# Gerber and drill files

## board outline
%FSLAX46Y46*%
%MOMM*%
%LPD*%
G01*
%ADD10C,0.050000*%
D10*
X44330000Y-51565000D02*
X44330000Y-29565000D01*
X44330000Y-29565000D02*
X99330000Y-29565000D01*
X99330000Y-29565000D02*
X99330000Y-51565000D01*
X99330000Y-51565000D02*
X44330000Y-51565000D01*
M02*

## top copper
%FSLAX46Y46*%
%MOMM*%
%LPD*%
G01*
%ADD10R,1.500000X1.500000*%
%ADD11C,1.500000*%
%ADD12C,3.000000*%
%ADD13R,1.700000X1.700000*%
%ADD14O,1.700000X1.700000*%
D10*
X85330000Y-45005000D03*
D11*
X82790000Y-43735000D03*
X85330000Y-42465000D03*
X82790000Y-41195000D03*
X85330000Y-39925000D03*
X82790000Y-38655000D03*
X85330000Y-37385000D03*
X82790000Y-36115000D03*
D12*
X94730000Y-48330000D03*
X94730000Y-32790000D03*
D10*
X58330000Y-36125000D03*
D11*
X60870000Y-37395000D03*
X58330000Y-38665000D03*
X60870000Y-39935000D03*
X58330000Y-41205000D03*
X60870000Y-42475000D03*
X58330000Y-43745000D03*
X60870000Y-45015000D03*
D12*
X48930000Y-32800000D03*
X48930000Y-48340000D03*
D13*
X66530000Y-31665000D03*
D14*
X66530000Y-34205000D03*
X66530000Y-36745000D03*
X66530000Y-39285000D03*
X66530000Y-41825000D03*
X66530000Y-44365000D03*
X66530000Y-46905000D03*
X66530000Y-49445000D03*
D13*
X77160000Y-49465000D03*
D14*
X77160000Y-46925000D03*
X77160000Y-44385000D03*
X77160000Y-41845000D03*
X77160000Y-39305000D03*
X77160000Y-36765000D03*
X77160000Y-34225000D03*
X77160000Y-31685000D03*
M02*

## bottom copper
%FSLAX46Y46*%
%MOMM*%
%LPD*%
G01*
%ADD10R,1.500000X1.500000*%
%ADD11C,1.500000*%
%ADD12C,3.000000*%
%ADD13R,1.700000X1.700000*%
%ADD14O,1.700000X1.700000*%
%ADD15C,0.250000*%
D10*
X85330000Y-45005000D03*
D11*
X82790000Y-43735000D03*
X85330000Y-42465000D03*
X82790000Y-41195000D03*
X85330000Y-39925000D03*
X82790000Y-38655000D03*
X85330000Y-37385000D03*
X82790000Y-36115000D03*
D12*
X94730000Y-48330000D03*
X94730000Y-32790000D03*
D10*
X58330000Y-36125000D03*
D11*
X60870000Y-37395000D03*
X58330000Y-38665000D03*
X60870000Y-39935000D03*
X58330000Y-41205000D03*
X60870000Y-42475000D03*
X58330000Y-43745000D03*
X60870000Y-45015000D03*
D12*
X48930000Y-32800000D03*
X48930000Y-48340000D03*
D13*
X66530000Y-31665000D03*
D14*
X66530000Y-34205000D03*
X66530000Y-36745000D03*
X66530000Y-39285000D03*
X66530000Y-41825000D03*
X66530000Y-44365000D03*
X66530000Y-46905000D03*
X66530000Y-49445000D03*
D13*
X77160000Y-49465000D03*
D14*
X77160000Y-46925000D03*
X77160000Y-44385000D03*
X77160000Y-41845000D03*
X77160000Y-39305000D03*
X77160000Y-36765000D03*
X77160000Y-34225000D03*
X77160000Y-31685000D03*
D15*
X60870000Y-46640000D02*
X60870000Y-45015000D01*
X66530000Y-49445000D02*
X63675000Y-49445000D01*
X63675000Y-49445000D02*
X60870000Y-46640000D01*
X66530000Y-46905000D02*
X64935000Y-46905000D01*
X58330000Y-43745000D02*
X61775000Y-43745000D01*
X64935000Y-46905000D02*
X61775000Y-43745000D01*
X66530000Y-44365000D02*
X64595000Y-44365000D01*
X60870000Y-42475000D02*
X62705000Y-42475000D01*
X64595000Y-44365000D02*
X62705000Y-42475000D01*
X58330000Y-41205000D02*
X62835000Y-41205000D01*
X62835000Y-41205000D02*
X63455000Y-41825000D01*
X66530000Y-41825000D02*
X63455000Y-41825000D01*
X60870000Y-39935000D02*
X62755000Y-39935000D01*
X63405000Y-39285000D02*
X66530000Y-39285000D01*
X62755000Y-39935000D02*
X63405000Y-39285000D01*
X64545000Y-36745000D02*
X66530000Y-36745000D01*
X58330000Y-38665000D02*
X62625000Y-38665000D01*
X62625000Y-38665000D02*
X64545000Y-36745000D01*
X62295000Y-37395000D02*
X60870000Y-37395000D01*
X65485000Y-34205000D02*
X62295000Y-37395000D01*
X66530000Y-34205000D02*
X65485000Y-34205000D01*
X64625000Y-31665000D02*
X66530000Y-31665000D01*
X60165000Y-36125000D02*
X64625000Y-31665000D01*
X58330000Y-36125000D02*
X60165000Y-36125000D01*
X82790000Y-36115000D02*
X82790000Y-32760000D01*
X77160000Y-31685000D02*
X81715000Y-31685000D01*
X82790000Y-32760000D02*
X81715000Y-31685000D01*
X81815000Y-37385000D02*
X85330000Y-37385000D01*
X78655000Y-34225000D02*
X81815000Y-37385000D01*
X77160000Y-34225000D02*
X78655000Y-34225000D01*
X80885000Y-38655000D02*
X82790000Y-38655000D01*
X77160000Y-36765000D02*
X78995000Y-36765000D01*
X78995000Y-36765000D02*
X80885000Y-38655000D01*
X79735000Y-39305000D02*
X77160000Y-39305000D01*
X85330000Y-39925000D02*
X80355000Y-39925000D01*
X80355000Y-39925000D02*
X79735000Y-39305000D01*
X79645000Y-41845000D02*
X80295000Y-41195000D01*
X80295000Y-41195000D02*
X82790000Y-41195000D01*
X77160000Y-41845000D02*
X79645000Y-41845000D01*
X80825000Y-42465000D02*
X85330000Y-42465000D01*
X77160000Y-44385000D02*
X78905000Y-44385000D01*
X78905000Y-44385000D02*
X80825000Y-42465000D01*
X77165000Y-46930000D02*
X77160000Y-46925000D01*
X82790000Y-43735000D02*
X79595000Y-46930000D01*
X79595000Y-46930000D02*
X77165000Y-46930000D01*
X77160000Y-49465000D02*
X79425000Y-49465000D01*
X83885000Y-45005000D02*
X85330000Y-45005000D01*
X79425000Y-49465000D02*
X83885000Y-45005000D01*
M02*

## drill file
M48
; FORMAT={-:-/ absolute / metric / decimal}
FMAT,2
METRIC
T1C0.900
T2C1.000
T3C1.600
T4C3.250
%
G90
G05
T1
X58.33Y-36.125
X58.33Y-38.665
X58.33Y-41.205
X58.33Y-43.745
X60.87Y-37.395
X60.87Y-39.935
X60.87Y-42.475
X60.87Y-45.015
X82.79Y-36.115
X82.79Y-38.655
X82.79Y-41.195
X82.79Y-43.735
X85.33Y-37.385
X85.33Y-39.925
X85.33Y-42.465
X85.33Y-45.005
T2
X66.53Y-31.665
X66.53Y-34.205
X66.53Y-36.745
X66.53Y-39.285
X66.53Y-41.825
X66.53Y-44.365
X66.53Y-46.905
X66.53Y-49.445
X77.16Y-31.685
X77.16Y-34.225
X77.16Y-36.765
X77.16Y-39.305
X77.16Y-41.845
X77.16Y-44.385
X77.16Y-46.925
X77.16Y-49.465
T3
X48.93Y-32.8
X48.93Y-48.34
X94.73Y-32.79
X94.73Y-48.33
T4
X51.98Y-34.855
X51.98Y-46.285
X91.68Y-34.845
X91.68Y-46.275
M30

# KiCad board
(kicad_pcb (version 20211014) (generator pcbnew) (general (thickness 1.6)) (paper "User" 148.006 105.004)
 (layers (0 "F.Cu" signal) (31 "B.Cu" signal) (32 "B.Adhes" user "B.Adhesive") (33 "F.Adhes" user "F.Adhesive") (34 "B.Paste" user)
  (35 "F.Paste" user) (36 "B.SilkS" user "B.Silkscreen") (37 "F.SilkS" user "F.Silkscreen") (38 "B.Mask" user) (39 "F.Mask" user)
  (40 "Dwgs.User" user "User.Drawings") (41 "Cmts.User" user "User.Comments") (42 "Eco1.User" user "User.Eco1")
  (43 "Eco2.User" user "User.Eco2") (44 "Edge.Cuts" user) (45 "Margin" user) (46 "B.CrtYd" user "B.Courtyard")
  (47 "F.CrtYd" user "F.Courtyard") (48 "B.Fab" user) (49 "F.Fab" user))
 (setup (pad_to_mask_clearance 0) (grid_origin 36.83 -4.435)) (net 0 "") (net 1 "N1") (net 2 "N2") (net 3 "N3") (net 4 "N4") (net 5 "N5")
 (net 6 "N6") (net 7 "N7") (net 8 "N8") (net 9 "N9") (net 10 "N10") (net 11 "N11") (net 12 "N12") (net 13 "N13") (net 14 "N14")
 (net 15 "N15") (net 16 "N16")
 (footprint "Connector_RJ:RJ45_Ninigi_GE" (layer "F.Cu") (at 85.33 45.005 90)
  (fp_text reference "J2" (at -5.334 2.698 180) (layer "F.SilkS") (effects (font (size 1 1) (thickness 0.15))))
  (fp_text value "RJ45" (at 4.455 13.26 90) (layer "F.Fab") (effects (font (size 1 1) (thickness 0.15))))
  (pad "" np_thru_hole circle locked (at -1.27 6.35 90) (size 3.25 3.25) (drill 3.25) (layers *.Cu *.Mask))
  (pad "" np_thru_hole circle locked (at 10.16 6.35 270) (size 3.25 3.25) (drill 3.25) (layers *.Cu *.Mask))
  (pad "1" thru_hole rect locked (at 0 0 270) (size 1.5 1.5) (drill 0.9) (layers *.Cu *.Mask) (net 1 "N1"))
  (pad "2" thru_hole circle locked (at 1.27 -2.54 270) (size 1.5 1.5) (drill 0.9) (layers *.Cu *.Mask) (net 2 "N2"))
  (pad "3" thru_hole circle locked (at 2.54 0 270) (size 1.5 1.5) (drill 0.9) (layers *.Cu *.Mask) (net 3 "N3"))
  (pad "4" thru_hole circle locked (at 3.81 -2.54 270) (size 1.5 1.5) (drill 0.9) (layers *.Cu *.Mask) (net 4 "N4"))
  (pad "5" thru_hole circle locked (at 5.08 0 270) (size 1.5 1.5) (drill 0.9) (layers *.Cu *.Mask) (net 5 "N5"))
  (pad "6" thru_hole circle locked (at 6.35 -2.54 270) (size 1.5 1.5) (drill 0.9) (layers *.Cu *.Mask) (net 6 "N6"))
  (pad "7" thru_hole circle locked (at 7.62 0 270) (size 1.5 1.5) (drill 0.9) (layers *.Cu *.Mask) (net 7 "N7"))
  (pad "8" thru_hole circle locked (at 8.89 -2.54 270) (size 1.5 1.5) (drill 0.9) (layers *.Cu *.Mask) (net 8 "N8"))
  (pad "SH" thru_hole circle locked (at -3.325 9.4 90) (size 3 3) (drill 1.6) (layers *.Cu *.Mask))
  (pad "SH" thru_hole circle locked (at 12.215 9.4 270) (size 3 3) (drill 1.6) (layers *.Cu *.Mask)))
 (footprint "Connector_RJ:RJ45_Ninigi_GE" (layer "F.Cu") (at 58.33 36.125 -90)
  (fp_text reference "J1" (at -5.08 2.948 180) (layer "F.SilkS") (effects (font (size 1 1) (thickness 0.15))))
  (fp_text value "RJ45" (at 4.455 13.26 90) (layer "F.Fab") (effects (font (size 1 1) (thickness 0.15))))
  (pad "" np_thru_hole circle locked (at 10.16 6.35 90) (size 3.25 3.25) (drill 3.25) (layers *.Cu *.Mask))
  (pad "" np_thru_hole circle locked (at -1.27 6.35 270) (size 3.25 3.25) (drill 3.25) (layers *.Cu *.Mask))
  (pad "1" thru_hole rect locked (at 0 0 90) (size 1.5 1.5) (drill 0.9) (layers *.Cu *.Mask) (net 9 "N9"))
  (pad "2" thru_hole circle locked (at 1.27 -2.54 90) (size 1.5 1.5) (drill 0.9) (layers *.Cu *.Mask) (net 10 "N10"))
  (pad "3" thru_hole circle locked (at 2.54 0 90) (size 1.5 1.5) (drill 0.9) (layers *.Cu *.Mask) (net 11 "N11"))
  (pad "4" thru_hole circle locked (at 3.81 -2.54 90) (size 1.5 1.5) (drill 0.9) (layers *.Cu *.Mask) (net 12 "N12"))
  (pad "5" thru_hole circle locked (at 5.08 0 90) (size 1.5 1.5) (drill 0.9) (layers *.Cu *.Mask) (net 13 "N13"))
  (pad "6" thru_hole circle locked (at 6.35 -2.54 90) (size 1.5 1.5) (drill 0.9) (layers *.Cu *.Mask) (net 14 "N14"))
  (pad "7" thru_hole circle locked (at 7.62 0 90) (size 1.5 1.5) (drill 0.9) (layers *.Cu *.Mask) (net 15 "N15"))
  (pad "8" thru_hole circle locked (at 8.89 -2.54 90) (size 1.5 1.5) (drill 0.9) (layers *.Cu *.Mask) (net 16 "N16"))
  (pad "SH" thru_hole circle locked (at -3.325 9.4 270) (size 3 3) (drill 1.6) (layers *.Cu *.Mask))
  (pad "SH" thru_hole circle locked (at 12.215 9.4 90) (size 3 3) (drill 1.6) (layers *.Cu *.Mask)))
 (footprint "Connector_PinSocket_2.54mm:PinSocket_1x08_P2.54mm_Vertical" (layer "F.Cu") (at 66.53 31.665)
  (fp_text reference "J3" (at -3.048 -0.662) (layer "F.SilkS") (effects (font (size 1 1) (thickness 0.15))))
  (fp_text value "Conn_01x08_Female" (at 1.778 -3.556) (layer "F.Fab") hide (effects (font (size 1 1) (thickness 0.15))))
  (pad "1" thru_hole rect locked (at 0 0) (size 1.7 1.7) (drill 1) (layers *.Cu *.Mask) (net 9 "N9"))
  (pad "2" thru_hole oval locked (at 0 2.54) (size 1.7 1.7) (drill 1) (layers *.Cu *.Mask) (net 10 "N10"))
  (pad "3" thru_hole oval locked (at 0 5.08) (size 1.7 1.7) (drill 1) (layers *.Cu *.Mask) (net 11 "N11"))
  (pad "4" thru_hole oval locked (at 0 7.62) (size 1.7 1.7) (drill 1) (layers *.Cu *.Mask) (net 12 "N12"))
  (pad "5" thru_hole oval locked (at 0 10.16) (size 1.7 1.7) (drill 1) (layers *.Cu *.Mask) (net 13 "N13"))
  (pad "6" thru_hole oval locked (at 0 12.7) (size 1.7 1.7) (drill 1) (layers *.Cu *.Mask) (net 14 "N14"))
  (pad "7" thru_hole oval locked (at 0 15.24) (size 1.7 1.7) (drill 1) (layers *.Cu *.Mask) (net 15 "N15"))
  (pad "8" thru_hole oval locked (at 0 17.78) (size 1.7 1.7) (drill 1) (layers *.Cu *.Mask) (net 16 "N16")))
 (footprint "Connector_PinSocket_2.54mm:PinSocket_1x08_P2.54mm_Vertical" (layer "F.Cu") (at 77.16 49.465 180)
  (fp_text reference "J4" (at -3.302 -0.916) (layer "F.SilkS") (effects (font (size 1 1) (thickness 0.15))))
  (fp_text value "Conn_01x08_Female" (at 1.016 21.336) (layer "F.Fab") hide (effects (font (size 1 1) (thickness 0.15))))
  (pad "1" thru_hole rect locked (at 0 0 180) (size 1.7 1.7) (drill 1) (layers *.Cu *.Mask) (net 1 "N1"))
  (pad "2" thru_hole oval locked (at 0 2.54 180) (size 1.7 1.7) (drill 1) (layers *.Cu *.Mask) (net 2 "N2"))
  (pad "3" thru_hole oval locked (at 0 5.08 180) (size 1.7 1.7) (drill 1) (layers *.Cu *.Mask) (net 3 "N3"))
  (pad "4" thru_hole oval locked (at 0 7.62 180) (size 1.7 1.7) (drill 1) (layers *.Cu *.Mask) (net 4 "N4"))
  (pad "5" thru_hole oval locked (at 0 10.16 180) (size 1.7 1.7) (drill 1) (layers *.Cu *.Mask) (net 5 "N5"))
  (pad "6" thru_hole oval locked (at 0 12.7 180) (size 1.7 1.7) (drill 1) (layers *.Cu *.Mask) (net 6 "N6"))
  (pad "7" thru_hole oval locked (at 0 15.24 180) (size 1.7 1.7) (drill 1) (layers *.Cu *.Mask) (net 7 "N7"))
  (pad "8" thru_hole oval locked (at 0 17.78 180) (size 1.7 1.7) (drill 1) (layers *.Cu *.Mask) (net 8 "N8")))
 (gr_line (start 44.33 51.565) (end 44.33 29.565) (layer "Edge.Cuts") (width 0.05))
 (gr_line (start 44.33 29.565) (end 99.33 29.565) (layer "Edge.Cuts") (width 0.05))
 (gr_line (start 99.33 29.565) (end 99.33 51.565) (layer "Edge.Cuts") (width 0.05))
 (gr_line (start 99.33 51.565) (end 44.33 51.565) (layer "Edge.Cuts") (width 0.05))
 (segment (start 60.87 46.64) (end 60.87 45.015) (width 0.25) (layer "B.Cu") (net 16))
 (segment (start 66.53 49.445) (end 63.675 49.445) (width 0.25) (layer "B.Cu") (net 16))
 (segment (start 63.675 49.445) (end 60.87 46.64) (width 0.25) (layer "B.Cu") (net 16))
 (segment (start 66.53 46.905) (end 64.935 46.905) (width 0.25) (layer "B.Cu") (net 15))
 (segment (start 58.33 43.745) (end 61.775 43.745) (width 0.25) (layer "B.Cu") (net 15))
 (segment (start 64.935 46.905) (end 61.775 43.745) (width 0.25) (layer "B.Cu") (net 15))
 (segment (start 66.53 44.365) (end 64.595 44.365) (width 0.25) (layer "B.Cu") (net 14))
 (segment (start 60.87 42.475) (end 62.705 42.475) (width 0.25) (layer "B.Cu") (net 14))
 (segment (start 64.595 44.365) (end 62.705 42.475) (width 0.25) (layer "B.Cu") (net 14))
 (segment (start 58.33 41.205) (end 62.835 41.205) (width 0.25) (layer "B.Cu") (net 13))
 (segment (start 62.835 41.205) (end 63.455 41.825) (width 0.25) (layer "B.Cu") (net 13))
 (segment (start 66.53 41.825) (end 63.455 41.825) (width 0.25) (layer "B.Cu") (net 13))
 (segment (start 60.87 39.935) (end 62.755 39.935) (width 0.25) (layer "B.Cu") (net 12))
 (segment (start 63.405 39.285) (end 66.53 39.285) (width 0.25) (layer "B.Cu") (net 12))
 (segment (start 62.755 39.935) (end 63.405 39.285) (width 0.25) (layer "B.Cu") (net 12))
 (segment (start 64.545 36.745) (end 66.53 36.745) (width 0.25) (layer "B.Cu") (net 11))
 (segment (start 58.33 38.665) (end 62.625 38.665) (width 0.25) (layer "B.Cu") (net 11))
 (segment (start 62.625 38.665) (end 64.545 36.745) (width 0.25) (layer "B.Cu") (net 11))
 (segment (start 62.295 37.395) (end 60.87 37.395) (width 0.25) (layer "B.Cu") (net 10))
 (segment (start 65.485 34.205) (end 62.295 37.395) (width 0.25) (layer "B.Cu") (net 10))
 (segment (start 66.53 34.205) (end 65.485 34.205) (width 0.25) (layer "B.Cu") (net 10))
 (segment (start 64.625 31.665) (end 66.53 31.665) (width 0.25) (layer "B.Cu") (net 9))
 (segment (start 60.165 36.125) (end 64.625 31.665) (width 0.25) (layer "B.Cu") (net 9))
 (segment (start 58.33 36.125) (end 60.165 36.125) (width 0.25) (layer "B.Cu") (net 9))
 (segment (start 82.79 36.115) (end 82.79 32.76) (width 0.25) (layer "B.Cu") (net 8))
 (segment (start 77.16 31.685) (end 81.715 31.685) (width 0.25) (layer "B.Cu") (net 8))
 (segment (start 82.79 32.76) (end 81.715 31.685) (width 0.25) (layer "B.Cu") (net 8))
 (segment (start 81.815 37.385) (end 85.33 37.385) (width 0.25) (layer "B.Cu") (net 7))
 (segment (start 78.655 34.225) (end 81.815 37.385) (width 0.25) (layer "B.Cu") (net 7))
 (segment (start 77.16 34.225) (end 78.655 34.225) (width 0.25) (layer "B.Cu") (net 7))
 (segment (start 80.885 38.655) (end 82.79 38.655) (width 0.25) (layer "B.Cu") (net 6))
 (segment (start 77.16 36.765) (end 78.995 36.765) (width 0.25) (layer "B.Cu") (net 6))
 (segment (start 78.995 36.765) (end 80.885 38.655) (width 0.25) (layer "B.Cu") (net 6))
 (segment (start 79.735 39.305) (end 77.16 39.305) (width 0.25) (layer "B.Cu") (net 5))
 (segment (start 85.33 39.925) (end 80.355 39.925) (width 0.25) (layer "B.Cu") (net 5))
 (segment (start 80.355 39.925) (end 79.735 39.305) (width 0.25) (layer "B.Cu") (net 5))
 (segment (start 79.645 41.845) (end 80.295 41.195) (width 0.25) (layer "B.Cu") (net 4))
 (segment (start 80.295 41.195) (end 82.79 41.195) (width 0.25) (layer "B.Cu") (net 4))
 (segment (start 77.16 41.845) (end 79.645 41.845) (width 0.25) (layer "B.Cu") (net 4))
 (segment (start 80.825 42.465) (end 85.33 42.465) (width 0.25) (layer "B.Cu") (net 3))
 (segment (start 77.16 44.385) (end 78.905 44.385) (width 0.25) (layer "B.Cu") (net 3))
 (segment (start 78.905 44.385) (end 80.825 42.465) (width 0.25) (layer "B.Cu") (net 3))
 (segment (start 77.165 46.93) (end 77.16 46.925) (width 0.25) (layer "B.Cu") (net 2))
 (segment (start 82.79 43.735) (end 79.595 46.93) (width 0.25) (layer "B.Cu") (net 2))
 (segment (start 79.595 46.93) (end 77.165 46.93) (width 0.25) (layer "B.Cu") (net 2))
 (segment (start 77.16 49.465) (end 79.425 49.465) (width 0.25) (layer "B.Cu") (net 1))
 (segment (start 83.885 45.005) (end 85.33 45.005) (width 0.25) (layer "B.Cu") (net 1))
 (segment (start 79.425 49.465) (end 83.885 45.005) (width 0.25) (layer "B.Cu") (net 1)))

